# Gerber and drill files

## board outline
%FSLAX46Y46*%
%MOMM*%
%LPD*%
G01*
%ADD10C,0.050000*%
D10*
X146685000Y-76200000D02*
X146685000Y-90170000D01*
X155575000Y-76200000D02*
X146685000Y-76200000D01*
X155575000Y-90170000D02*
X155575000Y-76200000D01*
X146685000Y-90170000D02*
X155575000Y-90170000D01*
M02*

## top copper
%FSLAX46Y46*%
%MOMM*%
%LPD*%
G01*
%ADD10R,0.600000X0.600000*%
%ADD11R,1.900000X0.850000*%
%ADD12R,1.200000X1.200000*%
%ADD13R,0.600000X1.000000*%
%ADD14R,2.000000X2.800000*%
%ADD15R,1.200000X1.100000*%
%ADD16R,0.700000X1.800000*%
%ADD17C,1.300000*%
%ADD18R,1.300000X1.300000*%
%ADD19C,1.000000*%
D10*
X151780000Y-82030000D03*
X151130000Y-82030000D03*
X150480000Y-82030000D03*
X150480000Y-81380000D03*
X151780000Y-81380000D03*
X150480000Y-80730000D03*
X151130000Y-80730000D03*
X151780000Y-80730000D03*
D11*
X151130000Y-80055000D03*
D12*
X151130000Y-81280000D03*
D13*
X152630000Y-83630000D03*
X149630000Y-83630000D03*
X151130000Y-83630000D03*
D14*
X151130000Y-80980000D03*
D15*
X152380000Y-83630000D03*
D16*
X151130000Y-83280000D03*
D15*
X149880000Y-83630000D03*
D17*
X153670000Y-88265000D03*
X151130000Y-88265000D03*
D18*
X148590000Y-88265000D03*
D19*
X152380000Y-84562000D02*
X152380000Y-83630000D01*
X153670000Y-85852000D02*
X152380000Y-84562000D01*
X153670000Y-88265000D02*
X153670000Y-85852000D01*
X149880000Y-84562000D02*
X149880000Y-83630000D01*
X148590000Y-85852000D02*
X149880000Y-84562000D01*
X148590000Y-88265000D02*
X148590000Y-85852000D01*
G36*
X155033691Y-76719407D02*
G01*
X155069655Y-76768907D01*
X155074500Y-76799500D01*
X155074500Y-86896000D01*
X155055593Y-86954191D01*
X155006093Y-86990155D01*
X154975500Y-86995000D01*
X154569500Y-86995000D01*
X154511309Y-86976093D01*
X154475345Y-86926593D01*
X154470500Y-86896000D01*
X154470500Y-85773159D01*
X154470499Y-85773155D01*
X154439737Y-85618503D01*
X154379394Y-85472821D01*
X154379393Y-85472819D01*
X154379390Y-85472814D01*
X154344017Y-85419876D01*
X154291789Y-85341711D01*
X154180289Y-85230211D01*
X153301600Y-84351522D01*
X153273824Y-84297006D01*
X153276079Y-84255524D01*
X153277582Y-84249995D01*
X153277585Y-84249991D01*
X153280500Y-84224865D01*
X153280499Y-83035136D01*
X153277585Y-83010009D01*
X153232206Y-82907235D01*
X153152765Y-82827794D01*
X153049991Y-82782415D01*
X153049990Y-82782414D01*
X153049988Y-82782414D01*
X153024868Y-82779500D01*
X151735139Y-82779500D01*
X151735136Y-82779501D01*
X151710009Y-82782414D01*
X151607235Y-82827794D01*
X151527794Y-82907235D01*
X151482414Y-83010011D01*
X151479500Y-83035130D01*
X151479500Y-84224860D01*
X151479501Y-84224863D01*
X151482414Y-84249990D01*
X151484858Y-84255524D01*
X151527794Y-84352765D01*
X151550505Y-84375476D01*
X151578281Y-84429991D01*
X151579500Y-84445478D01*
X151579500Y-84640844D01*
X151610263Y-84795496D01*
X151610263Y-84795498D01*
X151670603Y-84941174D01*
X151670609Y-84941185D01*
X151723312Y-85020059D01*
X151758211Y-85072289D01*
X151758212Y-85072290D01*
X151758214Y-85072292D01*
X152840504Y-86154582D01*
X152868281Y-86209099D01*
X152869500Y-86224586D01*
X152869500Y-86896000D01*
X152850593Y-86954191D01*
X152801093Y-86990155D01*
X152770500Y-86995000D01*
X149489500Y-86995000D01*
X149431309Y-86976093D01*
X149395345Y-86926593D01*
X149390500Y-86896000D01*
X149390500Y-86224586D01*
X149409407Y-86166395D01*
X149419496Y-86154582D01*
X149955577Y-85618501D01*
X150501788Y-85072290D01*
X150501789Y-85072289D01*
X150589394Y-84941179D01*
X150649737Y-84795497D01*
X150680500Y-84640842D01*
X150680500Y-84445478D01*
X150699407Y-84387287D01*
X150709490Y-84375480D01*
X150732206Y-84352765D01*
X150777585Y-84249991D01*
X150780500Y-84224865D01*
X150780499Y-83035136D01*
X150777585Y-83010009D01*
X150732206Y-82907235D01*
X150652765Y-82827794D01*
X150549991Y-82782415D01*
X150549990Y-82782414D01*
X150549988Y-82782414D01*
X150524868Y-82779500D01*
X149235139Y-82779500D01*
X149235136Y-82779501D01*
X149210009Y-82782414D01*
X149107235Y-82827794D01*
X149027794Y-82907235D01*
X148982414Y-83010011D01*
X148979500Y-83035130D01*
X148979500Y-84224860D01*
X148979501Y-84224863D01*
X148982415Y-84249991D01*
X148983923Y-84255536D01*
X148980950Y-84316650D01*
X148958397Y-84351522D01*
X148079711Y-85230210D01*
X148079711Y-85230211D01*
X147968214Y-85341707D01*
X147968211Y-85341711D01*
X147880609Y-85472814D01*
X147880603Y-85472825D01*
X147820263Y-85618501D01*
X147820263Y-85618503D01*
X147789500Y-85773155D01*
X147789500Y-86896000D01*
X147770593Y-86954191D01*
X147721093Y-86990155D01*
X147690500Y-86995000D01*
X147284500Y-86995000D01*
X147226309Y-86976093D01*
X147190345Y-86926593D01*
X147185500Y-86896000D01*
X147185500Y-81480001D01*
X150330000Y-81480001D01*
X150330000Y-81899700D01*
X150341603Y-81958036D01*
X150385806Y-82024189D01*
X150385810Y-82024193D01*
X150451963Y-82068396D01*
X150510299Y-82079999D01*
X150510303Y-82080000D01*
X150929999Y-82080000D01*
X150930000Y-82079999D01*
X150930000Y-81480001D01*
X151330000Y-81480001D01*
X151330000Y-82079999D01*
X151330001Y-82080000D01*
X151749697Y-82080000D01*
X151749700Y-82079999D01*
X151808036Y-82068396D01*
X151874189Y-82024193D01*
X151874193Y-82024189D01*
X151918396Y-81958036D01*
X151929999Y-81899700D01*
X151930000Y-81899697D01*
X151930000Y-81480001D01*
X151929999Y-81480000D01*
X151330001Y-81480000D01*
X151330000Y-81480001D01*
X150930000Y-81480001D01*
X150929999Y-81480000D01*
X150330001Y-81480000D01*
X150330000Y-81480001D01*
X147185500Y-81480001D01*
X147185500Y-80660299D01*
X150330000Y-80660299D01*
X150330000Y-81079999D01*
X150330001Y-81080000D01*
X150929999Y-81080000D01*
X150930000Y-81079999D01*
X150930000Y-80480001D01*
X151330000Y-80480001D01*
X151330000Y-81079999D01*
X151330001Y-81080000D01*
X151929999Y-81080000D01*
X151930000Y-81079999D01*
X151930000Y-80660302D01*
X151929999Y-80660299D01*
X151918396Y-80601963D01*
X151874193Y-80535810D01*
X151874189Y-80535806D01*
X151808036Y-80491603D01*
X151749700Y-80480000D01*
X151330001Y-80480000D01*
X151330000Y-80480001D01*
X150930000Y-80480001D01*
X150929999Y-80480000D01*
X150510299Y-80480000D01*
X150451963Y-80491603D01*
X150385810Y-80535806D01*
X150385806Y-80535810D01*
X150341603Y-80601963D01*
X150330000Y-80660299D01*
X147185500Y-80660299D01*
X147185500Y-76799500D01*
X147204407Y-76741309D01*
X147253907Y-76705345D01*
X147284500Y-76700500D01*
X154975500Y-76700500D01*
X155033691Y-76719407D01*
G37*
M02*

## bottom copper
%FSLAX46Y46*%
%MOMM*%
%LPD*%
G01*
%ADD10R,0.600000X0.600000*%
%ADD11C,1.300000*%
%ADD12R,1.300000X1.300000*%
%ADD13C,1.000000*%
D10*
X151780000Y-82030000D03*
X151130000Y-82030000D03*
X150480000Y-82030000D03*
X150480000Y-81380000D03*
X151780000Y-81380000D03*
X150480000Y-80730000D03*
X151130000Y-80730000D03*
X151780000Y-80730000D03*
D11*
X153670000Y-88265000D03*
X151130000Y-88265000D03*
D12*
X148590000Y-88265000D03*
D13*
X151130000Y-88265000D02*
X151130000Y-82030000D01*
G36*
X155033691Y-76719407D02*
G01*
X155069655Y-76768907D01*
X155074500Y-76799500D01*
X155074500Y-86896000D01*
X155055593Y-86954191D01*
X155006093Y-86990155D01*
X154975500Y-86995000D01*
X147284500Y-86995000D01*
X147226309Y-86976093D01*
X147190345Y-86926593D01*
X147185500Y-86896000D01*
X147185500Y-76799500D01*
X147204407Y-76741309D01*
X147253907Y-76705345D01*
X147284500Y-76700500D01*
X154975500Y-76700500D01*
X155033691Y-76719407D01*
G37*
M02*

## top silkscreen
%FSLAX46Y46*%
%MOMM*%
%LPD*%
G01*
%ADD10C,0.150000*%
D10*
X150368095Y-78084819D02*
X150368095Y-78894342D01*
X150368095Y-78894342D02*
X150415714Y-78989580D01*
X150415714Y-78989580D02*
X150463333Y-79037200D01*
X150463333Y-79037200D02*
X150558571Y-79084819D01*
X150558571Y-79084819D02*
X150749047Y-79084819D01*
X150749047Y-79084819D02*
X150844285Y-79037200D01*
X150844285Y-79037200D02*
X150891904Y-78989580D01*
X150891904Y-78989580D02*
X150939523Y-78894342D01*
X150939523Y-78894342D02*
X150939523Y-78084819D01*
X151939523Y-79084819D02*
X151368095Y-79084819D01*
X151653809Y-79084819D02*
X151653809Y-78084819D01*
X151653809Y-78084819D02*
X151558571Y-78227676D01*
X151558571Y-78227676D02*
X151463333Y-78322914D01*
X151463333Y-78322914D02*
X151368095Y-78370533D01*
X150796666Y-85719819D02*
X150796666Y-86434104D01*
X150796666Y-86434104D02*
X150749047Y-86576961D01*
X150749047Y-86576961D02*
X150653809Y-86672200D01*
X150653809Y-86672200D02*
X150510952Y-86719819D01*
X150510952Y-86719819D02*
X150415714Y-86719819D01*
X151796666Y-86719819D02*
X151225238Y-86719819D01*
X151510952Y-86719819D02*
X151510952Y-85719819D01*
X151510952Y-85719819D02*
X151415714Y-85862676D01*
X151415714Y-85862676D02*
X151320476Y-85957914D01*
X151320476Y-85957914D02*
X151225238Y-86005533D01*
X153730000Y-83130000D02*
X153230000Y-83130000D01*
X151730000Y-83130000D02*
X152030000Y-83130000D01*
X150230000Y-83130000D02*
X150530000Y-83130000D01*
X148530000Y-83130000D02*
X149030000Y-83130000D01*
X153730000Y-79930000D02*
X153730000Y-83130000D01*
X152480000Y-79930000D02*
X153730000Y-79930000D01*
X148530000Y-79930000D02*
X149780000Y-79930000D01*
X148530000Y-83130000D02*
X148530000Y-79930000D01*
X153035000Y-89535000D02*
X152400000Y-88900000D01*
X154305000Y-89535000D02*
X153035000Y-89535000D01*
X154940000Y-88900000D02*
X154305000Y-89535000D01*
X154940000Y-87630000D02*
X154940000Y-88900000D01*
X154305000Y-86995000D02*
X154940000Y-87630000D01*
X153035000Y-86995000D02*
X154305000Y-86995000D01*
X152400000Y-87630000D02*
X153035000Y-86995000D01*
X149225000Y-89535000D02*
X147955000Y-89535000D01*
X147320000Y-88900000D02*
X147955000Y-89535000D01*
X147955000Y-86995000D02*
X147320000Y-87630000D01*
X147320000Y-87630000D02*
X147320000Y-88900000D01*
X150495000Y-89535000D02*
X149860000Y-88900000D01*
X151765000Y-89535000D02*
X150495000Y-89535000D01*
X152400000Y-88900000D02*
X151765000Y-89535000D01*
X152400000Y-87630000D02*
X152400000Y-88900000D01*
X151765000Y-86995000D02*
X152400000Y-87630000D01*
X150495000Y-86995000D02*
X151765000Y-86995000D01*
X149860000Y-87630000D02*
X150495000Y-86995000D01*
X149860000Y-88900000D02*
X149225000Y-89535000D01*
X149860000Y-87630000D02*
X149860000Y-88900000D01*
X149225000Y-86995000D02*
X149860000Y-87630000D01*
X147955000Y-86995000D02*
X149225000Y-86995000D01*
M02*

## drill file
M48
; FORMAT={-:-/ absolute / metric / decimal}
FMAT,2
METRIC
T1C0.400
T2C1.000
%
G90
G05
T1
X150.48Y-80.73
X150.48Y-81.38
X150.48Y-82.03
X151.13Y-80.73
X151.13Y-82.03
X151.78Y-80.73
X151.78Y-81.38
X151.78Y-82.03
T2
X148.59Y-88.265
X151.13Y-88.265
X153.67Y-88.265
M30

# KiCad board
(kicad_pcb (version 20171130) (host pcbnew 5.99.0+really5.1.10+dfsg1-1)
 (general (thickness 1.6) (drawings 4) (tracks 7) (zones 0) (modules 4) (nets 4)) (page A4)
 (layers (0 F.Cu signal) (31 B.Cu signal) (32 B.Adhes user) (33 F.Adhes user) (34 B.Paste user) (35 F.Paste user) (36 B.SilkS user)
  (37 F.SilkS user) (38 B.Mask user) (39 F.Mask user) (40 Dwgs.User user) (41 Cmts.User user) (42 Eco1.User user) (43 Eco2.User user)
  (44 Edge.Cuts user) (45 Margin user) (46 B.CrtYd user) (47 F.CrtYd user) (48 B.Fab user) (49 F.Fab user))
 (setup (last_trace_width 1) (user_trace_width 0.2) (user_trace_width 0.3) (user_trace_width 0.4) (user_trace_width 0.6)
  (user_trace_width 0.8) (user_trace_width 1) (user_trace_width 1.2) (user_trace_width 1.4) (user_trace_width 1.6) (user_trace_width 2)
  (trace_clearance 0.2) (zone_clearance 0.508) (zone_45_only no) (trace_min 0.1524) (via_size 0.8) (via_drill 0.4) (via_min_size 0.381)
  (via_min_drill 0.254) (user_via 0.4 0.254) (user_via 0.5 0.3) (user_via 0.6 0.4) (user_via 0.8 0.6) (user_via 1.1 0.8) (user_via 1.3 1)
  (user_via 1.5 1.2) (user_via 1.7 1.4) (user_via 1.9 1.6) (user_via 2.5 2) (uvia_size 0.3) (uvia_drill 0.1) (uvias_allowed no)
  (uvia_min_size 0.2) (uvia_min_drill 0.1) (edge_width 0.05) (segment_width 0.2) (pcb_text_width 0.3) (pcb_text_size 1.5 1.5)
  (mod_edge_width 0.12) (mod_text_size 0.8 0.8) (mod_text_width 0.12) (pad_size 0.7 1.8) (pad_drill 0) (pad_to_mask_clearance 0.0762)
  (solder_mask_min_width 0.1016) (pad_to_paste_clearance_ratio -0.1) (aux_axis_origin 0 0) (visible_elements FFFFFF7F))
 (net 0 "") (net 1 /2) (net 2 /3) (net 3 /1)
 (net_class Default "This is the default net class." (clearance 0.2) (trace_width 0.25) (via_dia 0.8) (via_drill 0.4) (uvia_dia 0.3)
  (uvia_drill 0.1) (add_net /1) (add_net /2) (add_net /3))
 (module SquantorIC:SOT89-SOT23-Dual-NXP (layer F.Cu) (at 151.13 81.88)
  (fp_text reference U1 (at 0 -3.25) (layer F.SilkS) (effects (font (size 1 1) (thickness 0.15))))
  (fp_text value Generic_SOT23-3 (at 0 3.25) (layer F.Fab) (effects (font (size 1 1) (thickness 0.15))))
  (fp_line (start 2.6 1.25) (end 2.1 1.25) (layer F.SilkS) (width 0.15))
  (fp_line (start 0.6 1.25) (end 0.9 1.25) (layer F.SilkS) (width 0.15))
  (fp_line (start -0.9 1.25) (end -0.6 1.25) (layer F.SilkS) (width 0.15))
  (fp_line (start -2.6 1.25) (end -2.1 1.25) (layer F.SilkS) (width 0.15))
  (fp_line (start 2.6 -1.95) (end 2.6 1.25) (layer F.SilkS) (width 0.15))
  (fp_line (start 1.35 -1.95) (end 2.6 -1.95) (layer F.SilkS) (width 0.15))
  (fp_line (start -2.6 -1.95) (end -1.35 -1.95) (layer F.SilkS) (width 0.15))
  (fp_line (start -2.6 1.25) (end -2.6 -1.95) (layer F.SilkS) (width 0.15))
  (pad 2 thru_hole rect (at 0.65 0.15) (size 0.6 0.6) (drill 0.4) (layers *.Cu *.Mask) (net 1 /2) (zone_connect 2))
  (pad 2 thru_hole rect (at 0 0.15) (size 0.6 0.6) (drill 0.4) (layers *.Cu *.Mask) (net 1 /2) (zone_connect 2))
  (pad 2 thru_hole rect (at -0.65 0.15) (size 0.6 0.6) (drill 0.4) (layers *.Cu *.Mask) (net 1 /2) (zone_connect 2))
  (pad 2 thru_hole rect (at -0.65 -0.5) (size 0.6 0.6) (drill 0.4) (layers *.Cu *.Mask) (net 1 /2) (zone_connect 2))
  (pad 2 thru_hole rect (at 0.65 -0.5) (size 0.6 0.6) (drill 0.4) (layers *.Cu *.Mask) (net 1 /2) (zone_connect 2))
  (pad 2 thru_hole rect (at -0.65 -1.15 90) (size 0.6 0.6) (drill 0.4) (layers *.Cu *.Mask) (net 1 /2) (zone_connect 2))
  (pad 2 thru_hole rect (at 0 -1.15) (size 0.6 0.6) (drill 0.4) (layers *.Cu *.Mask) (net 1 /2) (zone_connect 2))
  (pad 2 thru_hole rect (at 0.65 -1.15) (size 0.6 0.6) (drill 0.4) (layers *.Cu *.Mask) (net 1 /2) (zone_connect 2))
  (pad 2 smd rect (at 0 -1.825) (size 1.9 0.85) (layers F.Cu F.Paste) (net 1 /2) (zone_connect 2))
  (pad 2 smd rect (at 0 -0.6) (size 1.2 1.2) (layers F.Cu F.Paste) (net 1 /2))
  (pad 3 smd rect (at 1.5 1.75) (size 0.6 1) (layers F.Cu F.Paste) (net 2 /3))
  (pad 1 smd rect (at -1.5 1.75) (size 0.6 1) (layers F.Cu F.Paste) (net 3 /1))
  (pad 2 smd rect (at 0 1.75) (size 0.6 1) (layers F.Cu F.Paste) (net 1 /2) (zone_connect 2))
  (pad 2 smd rect (at 0 -0.9) (size 2 2.8) (layers F.Cu F.Mask) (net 1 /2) (zone_connect 2))
  (pad 3 smd rect (at 1.25 1.75) (size 1.2 1.1) (layers F.Cu F.Mask) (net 2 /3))
  (pad 2 smd rect (at 0 1.4) (size 0.7 1.8) (layers F.Cu F.Mask) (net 1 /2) (zone_connect 2))
  (pad 1 smd rect (at -1.25 1.75) (size 1.2 1.1) (layers F.Cu F.Mask) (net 3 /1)))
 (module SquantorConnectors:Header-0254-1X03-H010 (layer F.Cu) (at 151.13 88.265)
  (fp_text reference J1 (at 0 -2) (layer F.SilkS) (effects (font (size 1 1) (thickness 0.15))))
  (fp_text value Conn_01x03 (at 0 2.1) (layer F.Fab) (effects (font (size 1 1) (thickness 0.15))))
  (fp_line (start 1.905 1.27) (end 1.27 0.635) (layer F.SilkS) (width 0.15))
  (fp_line (start 3.175 1.27) (end 1.905 1.27) (layer F.SilkS) (width 0.15))
  (fp_line (start 3.81 0.635) (end 3.175 1.27) (layer F.SilkS) (width 0.15))
  (fp_line (start 3.81 -0.635) (end 3.81 0.635) (layer F.SilkS) (width 0.15))
  (fp_line (start 3.175 -1.27) (end 3.81 -0.635) (layer F.SilkS) (width 0.15))
  (fp_line (start 1.905 -1.27) (end 3.175 -1.27) (layer F.SilkS) (width 0.15))
  (fp_line (start 1.27 -0.635) (end 1.905 -1.27) (layer F.SilkS) (width 0.15))
  (fp_line (start -1.905 1.27) (end -3.175 1.27) (layer F.SilkS) (width 0.15))
  (fp_line (start -3.81 0.635) (end -3.175 1.27) (layer F.SilkS) (width 0.15))
  (fp_line (start -3.175 -1.27) (end -3.81 -0.635) (layer F.SilkS) (width 0.15))
  (fp_line (start -3.81 -0.635) (end -3.81 0.635) (layer F.SilkS) (width 0.15))
  (fp_line (start -0.635 1.27) (end -1.27 0.635) (layer F.SilkS) (width 0.15))
  (fp_line (start 0.635 1.27) (end -0.635 1.27) (layer F.SilkS) (width 0.15))
  (fp_line (start 1.27 0.635) (end 0.635 1.27) (layer F.SilkS) (width 0.15))
  (fp_line (start 1.27 -0.635) (end 1.27 0.635) (layer F.SilkS) (width 0.15))
  (fp_line (start 0.635 -1.27) (end 1.27 -0.635) (layer F.SilkS) (width 0.15))
  (fp_line (start -0.635 -1.27) (end 0.635 -1.27) (layer F.SilkS) (width 0.15))
  (fp_line (start -1.27 -0.635) (end -0.635 -1.27) (layer F.SilkS) (width 0.15))
  (fp_line (start -1.27 0.635) (end -1.905 1.27) (layer F.SilkS) (width 0.15))
  (fp_line (start -1.27 -0.635) (end -1.27 0.635) (layer F.SilkS) (width 0.15))
  (fp_line (start -1.905 -1.27) (end -1.27 -0.635) (layer F.SilkS) (width 0.15))
  (fp_line (start -3.175 -1.27) (end -1.905 -1.27) (layer F.SilkS) (width 0.15))
  (pad 3 thru_hole circle (at 2.54 0 180) (size 1.3 1.3) (drill 1) (layers *.Cu *.Mask) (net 2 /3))
  (pad 2 thru_hole circle (at 0 0 180) (size 1.3 1.3) (drill 1) (layers *.Cu *.Mask) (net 1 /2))
  (pad 1 thru_hole rect (at -2.54 0 180) (size 1.3 1.3) (drill 1) (layers *.Cu *.Mask) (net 3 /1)))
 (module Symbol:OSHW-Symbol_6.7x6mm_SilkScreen (layer B.Cu) (at 151.3 82.5 180)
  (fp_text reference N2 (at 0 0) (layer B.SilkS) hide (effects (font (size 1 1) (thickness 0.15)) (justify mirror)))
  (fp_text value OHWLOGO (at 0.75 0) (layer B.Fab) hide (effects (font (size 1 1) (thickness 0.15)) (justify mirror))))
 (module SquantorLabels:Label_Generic (layer B.Cu) (at 152 86.3 180)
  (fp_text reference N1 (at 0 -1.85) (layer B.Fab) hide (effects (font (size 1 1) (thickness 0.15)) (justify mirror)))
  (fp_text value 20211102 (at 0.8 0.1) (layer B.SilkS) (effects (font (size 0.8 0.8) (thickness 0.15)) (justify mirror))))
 (gr_line (start 146.685 76.2) (end 146.685 90.17) (layer Edge.Cuts) (width 0.05))
 (gr_line (start 155.575 76.2) (end 146.685 76.2) (layer Edge.Cuts) (width 0.05))
 (gr_line (start 155.575 90.17) (end 155.575 76.2) (layer Edge.Cuts) (width 0.05))
 (gr_line (start 146.685 90.17) (end 155.575 90.17) (layer Edge.Cuts) (width 0.05))
 (segment (start 152.38 84.562) (end 152.38 83.63) (width 1) (layer F.Cu) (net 2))
 (segment (start 153.67 85.852) (end 152.38 84.562) (width 1) (layer F.Cu) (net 2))
 (segment (start 153.67 88.265) (end 153.67 85.852) (width 1) (layer F.Cu) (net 2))
 (segment (start 151.13 88.265) (end 151.13 82.03) (width 1) (layer B.Cu) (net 1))
 (segment (start 149.88 84.562) (end 149.88 83.63) (width 1) (layer F.Cu) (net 3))
 (segment (start 148.59 85.852) (end 149.88 84.562) (width 1) (layer F.Cu) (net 3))
 (segment (start 148.59 88.265) (end 148.59 85.852) (width 1) (layer F.Cu) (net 3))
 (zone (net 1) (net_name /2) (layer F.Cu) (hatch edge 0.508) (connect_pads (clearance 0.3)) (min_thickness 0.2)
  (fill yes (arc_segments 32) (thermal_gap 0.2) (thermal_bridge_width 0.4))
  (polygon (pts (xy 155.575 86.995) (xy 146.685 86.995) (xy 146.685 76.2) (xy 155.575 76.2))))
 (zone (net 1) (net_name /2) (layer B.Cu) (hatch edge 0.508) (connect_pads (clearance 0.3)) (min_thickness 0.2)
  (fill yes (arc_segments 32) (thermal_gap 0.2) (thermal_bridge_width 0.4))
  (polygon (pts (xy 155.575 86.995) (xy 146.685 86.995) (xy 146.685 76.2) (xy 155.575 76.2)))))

